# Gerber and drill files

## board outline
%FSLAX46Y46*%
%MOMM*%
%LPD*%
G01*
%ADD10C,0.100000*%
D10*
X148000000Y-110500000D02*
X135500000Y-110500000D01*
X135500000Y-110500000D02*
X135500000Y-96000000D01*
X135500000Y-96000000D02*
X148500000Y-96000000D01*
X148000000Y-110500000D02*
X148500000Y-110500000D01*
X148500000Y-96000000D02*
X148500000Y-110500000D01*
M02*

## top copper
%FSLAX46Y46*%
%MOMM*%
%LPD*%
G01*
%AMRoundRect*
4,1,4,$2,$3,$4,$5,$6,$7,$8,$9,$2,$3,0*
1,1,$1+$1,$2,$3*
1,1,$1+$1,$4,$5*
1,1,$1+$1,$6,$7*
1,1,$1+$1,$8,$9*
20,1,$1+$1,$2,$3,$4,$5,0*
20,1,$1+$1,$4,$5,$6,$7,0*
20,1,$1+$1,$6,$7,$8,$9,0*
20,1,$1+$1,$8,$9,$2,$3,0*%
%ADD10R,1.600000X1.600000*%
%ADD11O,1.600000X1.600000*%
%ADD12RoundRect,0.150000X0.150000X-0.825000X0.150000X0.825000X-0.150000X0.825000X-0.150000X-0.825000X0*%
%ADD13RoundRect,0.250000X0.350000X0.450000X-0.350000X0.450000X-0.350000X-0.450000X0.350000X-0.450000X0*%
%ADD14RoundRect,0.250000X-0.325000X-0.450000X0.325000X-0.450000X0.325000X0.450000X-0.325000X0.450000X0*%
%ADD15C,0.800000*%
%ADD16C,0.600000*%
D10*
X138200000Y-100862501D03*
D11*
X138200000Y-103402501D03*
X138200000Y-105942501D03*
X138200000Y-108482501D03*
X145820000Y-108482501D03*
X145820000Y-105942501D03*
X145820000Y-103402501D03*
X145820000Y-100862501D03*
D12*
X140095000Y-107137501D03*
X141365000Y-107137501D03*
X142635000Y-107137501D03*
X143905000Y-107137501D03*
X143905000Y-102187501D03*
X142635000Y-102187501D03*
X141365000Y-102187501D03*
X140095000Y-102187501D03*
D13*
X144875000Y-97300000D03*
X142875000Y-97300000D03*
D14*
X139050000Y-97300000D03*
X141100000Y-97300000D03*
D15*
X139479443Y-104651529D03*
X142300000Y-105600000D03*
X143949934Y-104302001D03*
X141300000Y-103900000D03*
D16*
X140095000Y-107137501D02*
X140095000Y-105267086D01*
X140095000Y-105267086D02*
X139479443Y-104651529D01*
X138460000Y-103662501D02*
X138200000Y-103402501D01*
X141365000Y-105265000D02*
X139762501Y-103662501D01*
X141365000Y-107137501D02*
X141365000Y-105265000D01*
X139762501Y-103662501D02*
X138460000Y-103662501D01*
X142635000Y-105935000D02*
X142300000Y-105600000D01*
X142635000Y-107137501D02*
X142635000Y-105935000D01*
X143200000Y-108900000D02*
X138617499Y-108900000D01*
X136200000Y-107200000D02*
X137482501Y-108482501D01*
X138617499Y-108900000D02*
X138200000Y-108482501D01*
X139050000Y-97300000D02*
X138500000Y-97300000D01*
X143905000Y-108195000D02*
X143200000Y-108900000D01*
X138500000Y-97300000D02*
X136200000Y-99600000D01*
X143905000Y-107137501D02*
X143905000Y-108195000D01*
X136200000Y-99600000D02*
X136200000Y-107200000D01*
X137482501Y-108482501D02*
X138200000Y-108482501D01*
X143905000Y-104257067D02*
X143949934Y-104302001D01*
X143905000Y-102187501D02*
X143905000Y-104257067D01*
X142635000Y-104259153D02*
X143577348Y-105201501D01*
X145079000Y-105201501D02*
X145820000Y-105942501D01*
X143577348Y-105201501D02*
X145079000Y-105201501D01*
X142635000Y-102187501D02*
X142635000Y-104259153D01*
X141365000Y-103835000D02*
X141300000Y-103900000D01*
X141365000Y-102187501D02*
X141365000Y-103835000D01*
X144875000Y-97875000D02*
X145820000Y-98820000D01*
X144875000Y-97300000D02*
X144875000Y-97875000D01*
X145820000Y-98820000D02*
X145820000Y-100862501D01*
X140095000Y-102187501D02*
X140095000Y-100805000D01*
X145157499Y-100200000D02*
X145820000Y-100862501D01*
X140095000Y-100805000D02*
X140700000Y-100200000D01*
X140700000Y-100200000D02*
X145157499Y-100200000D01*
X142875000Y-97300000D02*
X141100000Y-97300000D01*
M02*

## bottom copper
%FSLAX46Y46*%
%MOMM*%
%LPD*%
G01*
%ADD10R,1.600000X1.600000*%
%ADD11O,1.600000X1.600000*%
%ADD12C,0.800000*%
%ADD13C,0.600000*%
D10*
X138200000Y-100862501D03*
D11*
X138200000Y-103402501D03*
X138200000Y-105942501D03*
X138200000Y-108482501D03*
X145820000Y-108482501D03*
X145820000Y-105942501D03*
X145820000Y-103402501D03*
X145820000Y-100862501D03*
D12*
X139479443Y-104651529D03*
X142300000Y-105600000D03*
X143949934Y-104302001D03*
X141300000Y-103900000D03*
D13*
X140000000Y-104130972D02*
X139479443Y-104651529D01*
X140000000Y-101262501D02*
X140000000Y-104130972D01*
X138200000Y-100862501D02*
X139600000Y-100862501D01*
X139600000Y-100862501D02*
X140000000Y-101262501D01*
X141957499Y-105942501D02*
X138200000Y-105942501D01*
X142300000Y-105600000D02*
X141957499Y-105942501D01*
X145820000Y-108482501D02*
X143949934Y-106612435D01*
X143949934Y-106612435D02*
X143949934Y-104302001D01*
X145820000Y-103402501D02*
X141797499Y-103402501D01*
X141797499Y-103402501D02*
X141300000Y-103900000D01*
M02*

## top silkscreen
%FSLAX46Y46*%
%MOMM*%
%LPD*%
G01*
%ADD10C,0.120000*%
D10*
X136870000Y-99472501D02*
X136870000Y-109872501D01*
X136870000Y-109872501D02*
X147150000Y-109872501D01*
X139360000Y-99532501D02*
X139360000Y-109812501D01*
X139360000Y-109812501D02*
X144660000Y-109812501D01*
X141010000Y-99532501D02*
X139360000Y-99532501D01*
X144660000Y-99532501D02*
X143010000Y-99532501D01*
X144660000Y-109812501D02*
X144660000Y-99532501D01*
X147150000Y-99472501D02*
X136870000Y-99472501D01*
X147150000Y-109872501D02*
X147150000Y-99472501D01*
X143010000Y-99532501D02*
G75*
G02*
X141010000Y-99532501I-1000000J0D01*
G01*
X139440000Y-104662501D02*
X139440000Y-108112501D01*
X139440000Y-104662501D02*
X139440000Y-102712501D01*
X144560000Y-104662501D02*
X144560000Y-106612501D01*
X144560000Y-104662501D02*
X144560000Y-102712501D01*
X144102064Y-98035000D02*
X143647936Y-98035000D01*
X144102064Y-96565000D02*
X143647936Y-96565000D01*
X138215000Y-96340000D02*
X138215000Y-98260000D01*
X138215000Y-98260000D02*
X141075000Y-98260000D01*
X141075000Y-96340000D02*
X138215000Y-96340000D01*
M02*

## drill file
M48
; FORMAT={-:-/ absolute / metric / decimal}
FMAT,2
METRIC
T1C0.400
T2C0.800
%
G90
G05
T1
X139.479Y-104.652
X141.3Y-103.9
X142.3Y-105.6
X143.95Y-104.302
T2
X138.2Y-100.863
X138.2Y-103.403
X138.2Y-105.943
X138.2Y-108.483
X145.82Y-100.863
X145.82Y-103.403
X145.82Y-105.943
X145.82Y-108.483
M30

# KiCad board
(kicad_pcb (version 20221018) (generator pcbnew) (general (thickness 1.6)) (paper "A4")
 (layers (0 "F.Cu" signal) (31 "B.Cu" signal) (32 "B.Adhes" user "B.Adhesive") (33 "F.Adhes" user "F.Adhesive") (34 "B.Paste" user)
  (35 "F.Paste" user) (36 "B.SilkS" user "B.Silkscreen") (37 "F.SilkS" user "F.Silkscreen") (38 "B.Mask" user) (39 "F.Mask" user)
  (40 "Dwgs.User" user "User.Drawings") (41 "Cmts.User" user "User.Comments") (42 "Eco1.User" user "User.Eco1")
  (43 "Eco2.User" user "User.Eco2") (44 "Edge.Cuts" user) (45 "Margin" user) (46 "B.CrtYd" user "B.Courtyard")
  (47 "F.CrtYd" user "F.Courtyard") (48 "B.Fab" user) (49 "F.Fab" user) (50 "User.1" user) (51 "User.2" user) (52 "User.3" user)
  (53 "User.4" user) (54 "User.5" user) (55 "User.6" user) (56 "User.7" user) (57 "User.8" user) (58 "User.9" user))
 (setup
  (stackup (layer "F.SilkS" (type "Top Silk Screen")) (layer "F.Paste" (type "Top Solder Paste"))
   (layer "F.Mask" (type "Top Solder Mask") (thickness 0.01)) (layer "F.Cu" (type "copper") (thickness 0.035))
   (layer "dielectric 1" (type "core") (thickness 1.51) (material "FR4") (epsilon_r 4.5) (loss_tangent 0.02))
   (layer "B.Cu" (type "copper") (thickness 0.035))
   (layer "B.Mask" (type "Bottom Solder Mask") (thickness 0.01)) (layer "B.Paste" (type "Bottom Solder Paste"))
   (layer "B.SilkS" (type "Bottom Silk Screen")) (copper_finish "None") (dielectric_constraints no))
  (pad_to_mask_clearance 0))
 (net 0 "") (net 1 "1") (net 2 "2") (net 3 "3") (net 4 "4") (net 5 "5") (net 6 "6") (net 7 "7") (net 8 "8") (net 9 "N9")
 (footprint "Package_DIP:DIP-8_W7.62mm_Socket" (layer "F.Cu") (at 138.2 100.862501)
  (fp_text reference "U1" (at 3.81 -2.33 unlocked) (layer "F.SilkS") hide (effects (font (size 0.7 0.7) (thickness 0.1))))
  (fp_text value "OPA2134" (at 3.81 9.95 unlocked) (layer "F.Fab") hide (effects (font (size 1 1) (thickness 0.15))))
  (fp_line (start -1.33 -1.39) (end -1.33 9.01) (stroke (width 0.12) (type solid)) (layer "F.SilkS"))
  (fp_line (start -1.33 9.01) (end 8.95 9.01) (stroke (width 0.12) (type solid)) (layer "F.SilkS"))
  (fp_line (start 1.16 -1.33) (end 1.16 8.95) (stroke (width 0.12) (type solid)) (layer "F.SilkS"))
  (fp_line (start 1.16 8.95) (end 6.46 8.95) (stroke (width 0.12) (type solid)) (layer "F.SilkS"))
  (fp_line (start 2.81 -1.33) (end 1.16 -1.33) (stroke (width 0.12) (type solid)) (layer "F.SilkS"))
  (fp_line (start 6.46 -1.33) (end 4.81 -1.33) (stroke (width 0.12) (type solid)) (layer "F.SilkS"))
  (fp_line (start 6.46 8.95) (end 6.46 -1.33) (stroke (width 0.12) (type solid)) (layer "F.SilkS"))
  (fp_line (start 8.95 -1.39) (end -1.33 -1.39) (stroke (width 0.12) (type solid)) (layer "F.SilkS"))
  (fp_line (start 8.95 9.01) (end 8.95 -1.39) (stroke (width 0.12) (type solid)) (layer "F.SilkS"))
  (fp_arc (start 4.81 -1.33) (mid 3.81 -0.33) (end 2.81 -1.33) (stroke (width 0.12) (type solid)) (layer "F.SilkS"))
  (pad "1" thru_hole rect (at 0 0) (size 1.6 1.6) (drill 0.8) (layers "*.Cu" "*.Mask") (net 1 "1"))
  (pad "2" thru_hole oval (at 0 2.54) (size 1.6 1.6) (drill 0.8) (layers "*.Cu" "*.Mask") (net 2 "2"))
  (pad "3" thru_hole oval (at 0 5.08) (size 1.6 1.6) (drill 0.8) (layers "*.Cu" "*.Mask") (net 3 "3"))
  (pad "4" thru_hole oval (at 0 7.62) (size 1.6 1.6) (drill 0.8) (layers "*.Cu" "*.Mask") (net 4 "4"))
  (pad "5" thru_hole oval (at 7.62 7.62) (size 1.6 1.6) (drill 0.8) (layers "*.Cu" "*.Mask") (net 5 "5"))
  (pad "6" thru_hole oval (at 7.62 5.08) (size 1.6 1.6) (drill 0.8) (layers "*.Cu" "*.Mask") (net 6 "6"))
  (pad "7" thru_hole oval (at 7.62 2.54) (size 1.6 1.6) (drill 0.8) (layers "*.Cu" "*.Mask") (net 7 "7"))
  (pad "8" thru_hole oval (at 7.62 0) (size 1.6 1.6) (drill 0.8) (layers "*.Cu" "*.Mask") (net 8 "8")))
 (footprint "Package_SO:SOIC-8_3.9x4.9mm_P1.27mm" (layer "F.Cu") (at 142 104.662501 90)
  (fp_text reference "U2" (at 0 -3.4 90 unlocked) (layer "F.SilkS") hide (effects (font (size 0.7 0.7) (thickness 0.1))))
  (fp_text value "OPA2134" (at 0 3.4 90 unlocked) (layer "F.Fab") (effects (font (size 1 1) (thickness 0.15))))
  (fp_line (start 0 -2.56) (end -3.45 -2.56) (stroke (width 0.12) (type solid)) (layer "F.SilkS"))
  (fp_line (start 0 -2.56) (end 1.95 -2.56) (stroke (width 0.12) (type solid)) (layer "F.SilkS"))
  (fp_line (start 0 2.56) (end -1.95 2.56) (stroke (width 0.12) (type solid)) (layer "F.SilkS"))
  (fp_line (start 0 2.56) (end 1.95 2.56) (stroke (width 0.12) (type solid)) (layer "F.SilkS"))
  (pad "1" smd roundrect (at -2.475 -1.905 90) (size 1.95 0.6) (layers "F.Cu" "F.Paste" "F.Mask") (roundrect_rratio 0.25) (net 1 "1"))
  (pad "2" smd roundrect (at -2.475 -0.635 90) (size 1.95 0.6) (layers "F.Cu" "F.Paste" "F.Mask") (roundrect_rratio 0.25) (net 2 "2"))
  (pad "3" smd roundrect (at -2.475 0.635 90) (size 1.95 0.6) (layers "F.Cu" "F.Paste" "F.Mask") (roundrect_rratio 0.25) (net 3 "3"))
  (pad "4" smd roundrect (at -2.475 1.905 90) (size 1.95 0.6) (layers "F.Cu" "F.Paste" "F.Mask") (roundrect_rratio 0.25) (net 4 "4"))
  (pad "5" smd roundrect (at 2.475 1.905 90) (size 1.95 0.6) (layers "F.Cu" "F.Paste" "F.Mask") (roundrect_rratio 0.25) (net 5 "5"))
  (pad "6" smd roundrect (at 2.475 0.635 90) (size 1.95 0.6) (layers "F.Cu" "F.Paste" "F.Mask") (roundrect_rratio 0.25) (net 6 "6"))
  (pad "7" smd roundrect (at 2.475 -0.635 90) (size 1.95 0.6) (layers "F.Cu" "F.Paste" "F.Mask") (roundrect_rratio 0.25) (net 7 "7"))
  (pad "8" smd roundrect (at 2.475 -1.905 90) (size 1.95 0.6) (layers "F.Cu" "F.Paste" "F.Mask") (roundrect_rratio 0.25) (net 8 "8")))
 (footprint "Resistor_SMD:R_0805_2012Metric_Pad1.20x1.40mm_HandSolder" (layer "F.Cu") (at 143.875 97.3 180)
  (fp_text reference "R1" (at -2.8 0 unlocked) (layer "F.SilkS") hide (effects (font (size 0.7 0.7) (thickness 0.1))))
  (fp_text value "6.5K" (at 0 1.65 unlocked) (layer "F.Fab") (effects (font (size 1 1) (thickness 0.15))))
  (fp_line (start -0.227064 -0.735) (end 0.227064 -0.735) (stroke (width 0.12) (type solid)) (layer "F.SilkS"))
  (fp_line (start -0.227064 0.735) (end 0.227064 0.735) (stroke (width 0.12) (type solid)) (layer "F.SilkS"))
  (pad "1" smd roundrect (at -1 0 180) (size 1.2 1.4) (layers "F.Cu" "F.Paste" "F.Mask") (roundrect_rratio 0.2083333333) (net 8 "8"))
  (pad "2" smd roundrect (at 1 0 180) (size 1.2 1.4) (layers "F.Cu" "F.Paste" "F.Mask") (roundrect_rratio 0.2083333333) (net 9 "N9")))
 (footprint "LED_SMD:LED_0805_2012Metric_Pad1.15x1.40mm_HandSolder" (layer "F.Cu") (at 140.075 97.3)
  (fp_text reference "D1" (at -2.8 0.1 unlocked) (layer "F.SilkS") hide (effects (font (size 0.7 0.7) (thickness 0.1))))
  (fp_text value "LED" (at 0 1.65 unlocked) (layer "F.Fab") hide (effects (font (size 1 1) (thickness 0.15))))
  (fp_line (start -1.86 -0.96) (end -1.86 0.96) (stroke (width 0.12) (type solid)) (layer "F.SilkS"))
  (fp_line (start -1.86 0.96) (end 1 0.96) (stroke (width 0.12) (type solid)) (layer "F.SilkS"))
  (fp_line (start 1 -0.96) (end -1.86 -0.96) (stroke (width 0.12) (type solid)) (layer "F.SilkS"))
  (pad "1" smd roundrect (at -1.025 0) (size 1.15 1.4) (layers "F.Cu" "F.Paste" "F.Mask") (roundrect_rratio 0.2173913043) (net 4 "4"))
  (pad "2" smd roundrect (at 1.025 0) (size 1.15 1.4) (layers "F.Cu" "F.Paste" "F.Mask") (roundrect_rratio 0.2173913043) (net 9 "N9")))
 (gr_line (start 148 110.5) (end 135.5 110.5) (stroke (width 0.1) (type default)) (layer "Edge.Cuts"))
 (gr_line (start 135.5 110.5) (end 135.5 96) (stroke (width 0.1) (type default)) (layer "Edge.Cuts"))
 (gr_line (start 135.5 96) (end 148.5 96) (stroke (width 0.1) (type default)) (layer "Edge.Cuts"))
 (gr_line (start 148 110.5) (end 148.5 110.5) (stroke (width 0.1) (type default)) (layer "Edge.Cuts"))
 (gr_line (start 148.5 96) (end 148.5 110.5) (stroke (width 0.1) (type default)) (layer "Edge.Cuts"))
 (segment (start 140.095 107.137501) (end 140.095 105.267086) (width 0.6) (layer "F.Cu") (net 1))
 (segment (start 140.095 105.267086) (end 139.479443 104.651529) (width 0.6) (layer "F.Cu") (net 1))
 (via (at 139.479443 104.651529) (size 0.8) (drill 0.4) (layers "F.Cu" "B.Cu") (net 1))
 (segment (start 140 104.130972) (end 139.479443 104.651529) (width 0.6) (layer "B.Cu") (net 1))
 (segment (start 140 101.262501) (end 140 104.130972) (width 0.6) (layer "B.Cu") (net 1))
 (segment (start 138.2 100.862501) (end 139.6 100.862501) (width 0.6) (layer "B.Cu") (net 1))
 (segment (start 139.6 100.862501) (end 140 101.262501) (width 0.6) (layer "B.Cu") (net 1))
 (segment (start 138.46 103.662501) (end 138.2 103.402501) (width 0.6) (layer "F.Cu") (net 2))
 (segment (start 141.365 105.265) (end 139.762501 103.662501) (width 0.6) (layer "F.Cu") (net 2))
 (segment (start 141.365 107.137501) (end 141.365 105.265) (width 0.6) (layer "F.Cu") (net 2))
 (segment (start 139.762501 103.662501) (end 138.46 103.662501) (width 0.6) (layer "F.Cu") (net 2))
 (segment (start 142.635 105.935) (end 142.3 105.6) (width 0.6) (layer "F.Cu") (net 3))
 (segment (start 142.635 107.137501) (end 142.635 105.935) (width 0.6) (layer "F.Cu") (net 3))
 (via (at 142.3 105.6) (size 0.8) (drill 0.4) (layers "F.Cu" "B.Cu") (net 3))
 (segment (start 141.957499 105.942501) (end 138.2 105.942501) (width 0.6) (layer "B.Cu") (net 3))
 (segment (start 142.3 105.6) (end 141.957499 105.942501) (width 0.6) (layer "B.Cu") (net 3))
 (segment (start 143.2 108.9) (end 138.617499 108.9) (width 0.6) (layer "F.Cu") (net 4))
 (segment (start 136.2 107.2) (end 137.482501 108.482501) (width 0.6) (layer "F.Cu") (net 4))
 (segment (start 138.617499 108.9) (end 138.2 108.482501) (width 0.6) (layer "F.Cu") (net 4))
 (segment (start 139.05 97.3) (end 138.5 97.3) (width 0.6) (layer "F.Cu") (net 4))
 (segment (start 143.905 108.195) (end 143.2 108.9) (width 0.6) (layer "F.Cu") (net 4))
 (segment (start 138.5 97.3) (end 136.2 99.6) (width 0.6) (layer "F.Cu") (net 4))
 (segment (start 143.905 107.137501) (end 143.905 108.195) (width 0.6) (layer "F.Cu") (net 4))
 (segment (start 136.2 99.6) (end 136.2 107.2) (width 0.6) (layer "F.Cu") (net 4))
 (segment (start 137.482501 108.482501) (end 138.2 108.482501) (width 0.6) (layer "F.Cu") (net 4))
 (segment (start 143.905 104.257067) (end 143.949934 104.302001) (width 0.6) (layer "F.Cu") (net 5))
 (segment (start 143.905 102.187501) (end 143.905 104.257067) (width 0.6) (layer "F.Cu") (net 5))
 (via (at 143.949934 104.302001) (size 0.8) (drill 0.4) (layers "F.Cu" "B.Cu") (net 5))
 (segment (start 145.82 108.482501) (end 143.949934 106.612435) (width 0.6) (layer "B.Cu") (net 5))
 (segment (start 143.949934 106.612435) (end 143.949934 104.302001) (width 0.6) (layer "B.Cu") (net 5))
 (segment (start 142.635 104.259153) (end 143.577348 105.201501) (width 0.6) (layer "F.Cu") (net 6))
 (segment (start 145.079 105.201501) (end 145.82 105.942501) (width 0.6) (layer "F.Cu") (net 6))
 (segment (start 143.577348 105.201501) (end 145.079 105.201501) (width 0.6) (layer "F.Cu") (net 6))
 (segment (start 142.635 102.187501) (end 142.635 104.259153) (width 0.6) (layer "F.Cu") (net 6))
 (segment (start 141.365 103.835) (end 141.3 103.9) (width 0.6) (layer "F.Cu") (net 7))
 (segment (start 141.365 102.187501) (end 141.365 103.835) (width 0.6) (layer "F.Cu") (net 7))
 (via (at 141.3 103.9) (size 0.8) (drill 0.4) (layers "F.Cu" "B.Cu") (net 7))
 (segment (start 145.82 103.402501) (end 141.797499 103.402501) (width 0.6) (layer "B.Cu") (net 7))
 (segment (start 141.797499 103.402501) (end 141.3 103.9) (width 0.6) (layer "B.Cu") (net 7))
 (segment (start 144.875 97.875) (end 145.82 98.82) (width 0.6) (layer "F.Cu") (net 8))
 (segment (start 144.875 97.3) (end 144.875 97.875) (width 0.6) (layer "F.Cu") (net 8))
 (segment (start 145.82 98.82) (end 145.82 100.862501) (width 0.6) (layer "F.Cu") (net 8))
 (segment (start 140.095 102.187501) (end 140.095 100.805) (width 0.6) (layer "F.Cu") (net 8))
 (segment (start 145.157499 100.2) (end 145.82 100.862501) (width 0.6) (layer "F.Cu") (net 8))
 (segment (start 140.095 100.805) (end 140.7 100.2) (width 0.6) (layer "F.Cu") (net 8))
 (segment (start 140.7 100.2) (end 145.157499 100.2) (width 0.6) (layer "F.Cu") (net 8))
 (segment (start 142.875 97.3) (end 141.1 97.3) (width 0.6) (layer "F.Cu") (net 9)))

